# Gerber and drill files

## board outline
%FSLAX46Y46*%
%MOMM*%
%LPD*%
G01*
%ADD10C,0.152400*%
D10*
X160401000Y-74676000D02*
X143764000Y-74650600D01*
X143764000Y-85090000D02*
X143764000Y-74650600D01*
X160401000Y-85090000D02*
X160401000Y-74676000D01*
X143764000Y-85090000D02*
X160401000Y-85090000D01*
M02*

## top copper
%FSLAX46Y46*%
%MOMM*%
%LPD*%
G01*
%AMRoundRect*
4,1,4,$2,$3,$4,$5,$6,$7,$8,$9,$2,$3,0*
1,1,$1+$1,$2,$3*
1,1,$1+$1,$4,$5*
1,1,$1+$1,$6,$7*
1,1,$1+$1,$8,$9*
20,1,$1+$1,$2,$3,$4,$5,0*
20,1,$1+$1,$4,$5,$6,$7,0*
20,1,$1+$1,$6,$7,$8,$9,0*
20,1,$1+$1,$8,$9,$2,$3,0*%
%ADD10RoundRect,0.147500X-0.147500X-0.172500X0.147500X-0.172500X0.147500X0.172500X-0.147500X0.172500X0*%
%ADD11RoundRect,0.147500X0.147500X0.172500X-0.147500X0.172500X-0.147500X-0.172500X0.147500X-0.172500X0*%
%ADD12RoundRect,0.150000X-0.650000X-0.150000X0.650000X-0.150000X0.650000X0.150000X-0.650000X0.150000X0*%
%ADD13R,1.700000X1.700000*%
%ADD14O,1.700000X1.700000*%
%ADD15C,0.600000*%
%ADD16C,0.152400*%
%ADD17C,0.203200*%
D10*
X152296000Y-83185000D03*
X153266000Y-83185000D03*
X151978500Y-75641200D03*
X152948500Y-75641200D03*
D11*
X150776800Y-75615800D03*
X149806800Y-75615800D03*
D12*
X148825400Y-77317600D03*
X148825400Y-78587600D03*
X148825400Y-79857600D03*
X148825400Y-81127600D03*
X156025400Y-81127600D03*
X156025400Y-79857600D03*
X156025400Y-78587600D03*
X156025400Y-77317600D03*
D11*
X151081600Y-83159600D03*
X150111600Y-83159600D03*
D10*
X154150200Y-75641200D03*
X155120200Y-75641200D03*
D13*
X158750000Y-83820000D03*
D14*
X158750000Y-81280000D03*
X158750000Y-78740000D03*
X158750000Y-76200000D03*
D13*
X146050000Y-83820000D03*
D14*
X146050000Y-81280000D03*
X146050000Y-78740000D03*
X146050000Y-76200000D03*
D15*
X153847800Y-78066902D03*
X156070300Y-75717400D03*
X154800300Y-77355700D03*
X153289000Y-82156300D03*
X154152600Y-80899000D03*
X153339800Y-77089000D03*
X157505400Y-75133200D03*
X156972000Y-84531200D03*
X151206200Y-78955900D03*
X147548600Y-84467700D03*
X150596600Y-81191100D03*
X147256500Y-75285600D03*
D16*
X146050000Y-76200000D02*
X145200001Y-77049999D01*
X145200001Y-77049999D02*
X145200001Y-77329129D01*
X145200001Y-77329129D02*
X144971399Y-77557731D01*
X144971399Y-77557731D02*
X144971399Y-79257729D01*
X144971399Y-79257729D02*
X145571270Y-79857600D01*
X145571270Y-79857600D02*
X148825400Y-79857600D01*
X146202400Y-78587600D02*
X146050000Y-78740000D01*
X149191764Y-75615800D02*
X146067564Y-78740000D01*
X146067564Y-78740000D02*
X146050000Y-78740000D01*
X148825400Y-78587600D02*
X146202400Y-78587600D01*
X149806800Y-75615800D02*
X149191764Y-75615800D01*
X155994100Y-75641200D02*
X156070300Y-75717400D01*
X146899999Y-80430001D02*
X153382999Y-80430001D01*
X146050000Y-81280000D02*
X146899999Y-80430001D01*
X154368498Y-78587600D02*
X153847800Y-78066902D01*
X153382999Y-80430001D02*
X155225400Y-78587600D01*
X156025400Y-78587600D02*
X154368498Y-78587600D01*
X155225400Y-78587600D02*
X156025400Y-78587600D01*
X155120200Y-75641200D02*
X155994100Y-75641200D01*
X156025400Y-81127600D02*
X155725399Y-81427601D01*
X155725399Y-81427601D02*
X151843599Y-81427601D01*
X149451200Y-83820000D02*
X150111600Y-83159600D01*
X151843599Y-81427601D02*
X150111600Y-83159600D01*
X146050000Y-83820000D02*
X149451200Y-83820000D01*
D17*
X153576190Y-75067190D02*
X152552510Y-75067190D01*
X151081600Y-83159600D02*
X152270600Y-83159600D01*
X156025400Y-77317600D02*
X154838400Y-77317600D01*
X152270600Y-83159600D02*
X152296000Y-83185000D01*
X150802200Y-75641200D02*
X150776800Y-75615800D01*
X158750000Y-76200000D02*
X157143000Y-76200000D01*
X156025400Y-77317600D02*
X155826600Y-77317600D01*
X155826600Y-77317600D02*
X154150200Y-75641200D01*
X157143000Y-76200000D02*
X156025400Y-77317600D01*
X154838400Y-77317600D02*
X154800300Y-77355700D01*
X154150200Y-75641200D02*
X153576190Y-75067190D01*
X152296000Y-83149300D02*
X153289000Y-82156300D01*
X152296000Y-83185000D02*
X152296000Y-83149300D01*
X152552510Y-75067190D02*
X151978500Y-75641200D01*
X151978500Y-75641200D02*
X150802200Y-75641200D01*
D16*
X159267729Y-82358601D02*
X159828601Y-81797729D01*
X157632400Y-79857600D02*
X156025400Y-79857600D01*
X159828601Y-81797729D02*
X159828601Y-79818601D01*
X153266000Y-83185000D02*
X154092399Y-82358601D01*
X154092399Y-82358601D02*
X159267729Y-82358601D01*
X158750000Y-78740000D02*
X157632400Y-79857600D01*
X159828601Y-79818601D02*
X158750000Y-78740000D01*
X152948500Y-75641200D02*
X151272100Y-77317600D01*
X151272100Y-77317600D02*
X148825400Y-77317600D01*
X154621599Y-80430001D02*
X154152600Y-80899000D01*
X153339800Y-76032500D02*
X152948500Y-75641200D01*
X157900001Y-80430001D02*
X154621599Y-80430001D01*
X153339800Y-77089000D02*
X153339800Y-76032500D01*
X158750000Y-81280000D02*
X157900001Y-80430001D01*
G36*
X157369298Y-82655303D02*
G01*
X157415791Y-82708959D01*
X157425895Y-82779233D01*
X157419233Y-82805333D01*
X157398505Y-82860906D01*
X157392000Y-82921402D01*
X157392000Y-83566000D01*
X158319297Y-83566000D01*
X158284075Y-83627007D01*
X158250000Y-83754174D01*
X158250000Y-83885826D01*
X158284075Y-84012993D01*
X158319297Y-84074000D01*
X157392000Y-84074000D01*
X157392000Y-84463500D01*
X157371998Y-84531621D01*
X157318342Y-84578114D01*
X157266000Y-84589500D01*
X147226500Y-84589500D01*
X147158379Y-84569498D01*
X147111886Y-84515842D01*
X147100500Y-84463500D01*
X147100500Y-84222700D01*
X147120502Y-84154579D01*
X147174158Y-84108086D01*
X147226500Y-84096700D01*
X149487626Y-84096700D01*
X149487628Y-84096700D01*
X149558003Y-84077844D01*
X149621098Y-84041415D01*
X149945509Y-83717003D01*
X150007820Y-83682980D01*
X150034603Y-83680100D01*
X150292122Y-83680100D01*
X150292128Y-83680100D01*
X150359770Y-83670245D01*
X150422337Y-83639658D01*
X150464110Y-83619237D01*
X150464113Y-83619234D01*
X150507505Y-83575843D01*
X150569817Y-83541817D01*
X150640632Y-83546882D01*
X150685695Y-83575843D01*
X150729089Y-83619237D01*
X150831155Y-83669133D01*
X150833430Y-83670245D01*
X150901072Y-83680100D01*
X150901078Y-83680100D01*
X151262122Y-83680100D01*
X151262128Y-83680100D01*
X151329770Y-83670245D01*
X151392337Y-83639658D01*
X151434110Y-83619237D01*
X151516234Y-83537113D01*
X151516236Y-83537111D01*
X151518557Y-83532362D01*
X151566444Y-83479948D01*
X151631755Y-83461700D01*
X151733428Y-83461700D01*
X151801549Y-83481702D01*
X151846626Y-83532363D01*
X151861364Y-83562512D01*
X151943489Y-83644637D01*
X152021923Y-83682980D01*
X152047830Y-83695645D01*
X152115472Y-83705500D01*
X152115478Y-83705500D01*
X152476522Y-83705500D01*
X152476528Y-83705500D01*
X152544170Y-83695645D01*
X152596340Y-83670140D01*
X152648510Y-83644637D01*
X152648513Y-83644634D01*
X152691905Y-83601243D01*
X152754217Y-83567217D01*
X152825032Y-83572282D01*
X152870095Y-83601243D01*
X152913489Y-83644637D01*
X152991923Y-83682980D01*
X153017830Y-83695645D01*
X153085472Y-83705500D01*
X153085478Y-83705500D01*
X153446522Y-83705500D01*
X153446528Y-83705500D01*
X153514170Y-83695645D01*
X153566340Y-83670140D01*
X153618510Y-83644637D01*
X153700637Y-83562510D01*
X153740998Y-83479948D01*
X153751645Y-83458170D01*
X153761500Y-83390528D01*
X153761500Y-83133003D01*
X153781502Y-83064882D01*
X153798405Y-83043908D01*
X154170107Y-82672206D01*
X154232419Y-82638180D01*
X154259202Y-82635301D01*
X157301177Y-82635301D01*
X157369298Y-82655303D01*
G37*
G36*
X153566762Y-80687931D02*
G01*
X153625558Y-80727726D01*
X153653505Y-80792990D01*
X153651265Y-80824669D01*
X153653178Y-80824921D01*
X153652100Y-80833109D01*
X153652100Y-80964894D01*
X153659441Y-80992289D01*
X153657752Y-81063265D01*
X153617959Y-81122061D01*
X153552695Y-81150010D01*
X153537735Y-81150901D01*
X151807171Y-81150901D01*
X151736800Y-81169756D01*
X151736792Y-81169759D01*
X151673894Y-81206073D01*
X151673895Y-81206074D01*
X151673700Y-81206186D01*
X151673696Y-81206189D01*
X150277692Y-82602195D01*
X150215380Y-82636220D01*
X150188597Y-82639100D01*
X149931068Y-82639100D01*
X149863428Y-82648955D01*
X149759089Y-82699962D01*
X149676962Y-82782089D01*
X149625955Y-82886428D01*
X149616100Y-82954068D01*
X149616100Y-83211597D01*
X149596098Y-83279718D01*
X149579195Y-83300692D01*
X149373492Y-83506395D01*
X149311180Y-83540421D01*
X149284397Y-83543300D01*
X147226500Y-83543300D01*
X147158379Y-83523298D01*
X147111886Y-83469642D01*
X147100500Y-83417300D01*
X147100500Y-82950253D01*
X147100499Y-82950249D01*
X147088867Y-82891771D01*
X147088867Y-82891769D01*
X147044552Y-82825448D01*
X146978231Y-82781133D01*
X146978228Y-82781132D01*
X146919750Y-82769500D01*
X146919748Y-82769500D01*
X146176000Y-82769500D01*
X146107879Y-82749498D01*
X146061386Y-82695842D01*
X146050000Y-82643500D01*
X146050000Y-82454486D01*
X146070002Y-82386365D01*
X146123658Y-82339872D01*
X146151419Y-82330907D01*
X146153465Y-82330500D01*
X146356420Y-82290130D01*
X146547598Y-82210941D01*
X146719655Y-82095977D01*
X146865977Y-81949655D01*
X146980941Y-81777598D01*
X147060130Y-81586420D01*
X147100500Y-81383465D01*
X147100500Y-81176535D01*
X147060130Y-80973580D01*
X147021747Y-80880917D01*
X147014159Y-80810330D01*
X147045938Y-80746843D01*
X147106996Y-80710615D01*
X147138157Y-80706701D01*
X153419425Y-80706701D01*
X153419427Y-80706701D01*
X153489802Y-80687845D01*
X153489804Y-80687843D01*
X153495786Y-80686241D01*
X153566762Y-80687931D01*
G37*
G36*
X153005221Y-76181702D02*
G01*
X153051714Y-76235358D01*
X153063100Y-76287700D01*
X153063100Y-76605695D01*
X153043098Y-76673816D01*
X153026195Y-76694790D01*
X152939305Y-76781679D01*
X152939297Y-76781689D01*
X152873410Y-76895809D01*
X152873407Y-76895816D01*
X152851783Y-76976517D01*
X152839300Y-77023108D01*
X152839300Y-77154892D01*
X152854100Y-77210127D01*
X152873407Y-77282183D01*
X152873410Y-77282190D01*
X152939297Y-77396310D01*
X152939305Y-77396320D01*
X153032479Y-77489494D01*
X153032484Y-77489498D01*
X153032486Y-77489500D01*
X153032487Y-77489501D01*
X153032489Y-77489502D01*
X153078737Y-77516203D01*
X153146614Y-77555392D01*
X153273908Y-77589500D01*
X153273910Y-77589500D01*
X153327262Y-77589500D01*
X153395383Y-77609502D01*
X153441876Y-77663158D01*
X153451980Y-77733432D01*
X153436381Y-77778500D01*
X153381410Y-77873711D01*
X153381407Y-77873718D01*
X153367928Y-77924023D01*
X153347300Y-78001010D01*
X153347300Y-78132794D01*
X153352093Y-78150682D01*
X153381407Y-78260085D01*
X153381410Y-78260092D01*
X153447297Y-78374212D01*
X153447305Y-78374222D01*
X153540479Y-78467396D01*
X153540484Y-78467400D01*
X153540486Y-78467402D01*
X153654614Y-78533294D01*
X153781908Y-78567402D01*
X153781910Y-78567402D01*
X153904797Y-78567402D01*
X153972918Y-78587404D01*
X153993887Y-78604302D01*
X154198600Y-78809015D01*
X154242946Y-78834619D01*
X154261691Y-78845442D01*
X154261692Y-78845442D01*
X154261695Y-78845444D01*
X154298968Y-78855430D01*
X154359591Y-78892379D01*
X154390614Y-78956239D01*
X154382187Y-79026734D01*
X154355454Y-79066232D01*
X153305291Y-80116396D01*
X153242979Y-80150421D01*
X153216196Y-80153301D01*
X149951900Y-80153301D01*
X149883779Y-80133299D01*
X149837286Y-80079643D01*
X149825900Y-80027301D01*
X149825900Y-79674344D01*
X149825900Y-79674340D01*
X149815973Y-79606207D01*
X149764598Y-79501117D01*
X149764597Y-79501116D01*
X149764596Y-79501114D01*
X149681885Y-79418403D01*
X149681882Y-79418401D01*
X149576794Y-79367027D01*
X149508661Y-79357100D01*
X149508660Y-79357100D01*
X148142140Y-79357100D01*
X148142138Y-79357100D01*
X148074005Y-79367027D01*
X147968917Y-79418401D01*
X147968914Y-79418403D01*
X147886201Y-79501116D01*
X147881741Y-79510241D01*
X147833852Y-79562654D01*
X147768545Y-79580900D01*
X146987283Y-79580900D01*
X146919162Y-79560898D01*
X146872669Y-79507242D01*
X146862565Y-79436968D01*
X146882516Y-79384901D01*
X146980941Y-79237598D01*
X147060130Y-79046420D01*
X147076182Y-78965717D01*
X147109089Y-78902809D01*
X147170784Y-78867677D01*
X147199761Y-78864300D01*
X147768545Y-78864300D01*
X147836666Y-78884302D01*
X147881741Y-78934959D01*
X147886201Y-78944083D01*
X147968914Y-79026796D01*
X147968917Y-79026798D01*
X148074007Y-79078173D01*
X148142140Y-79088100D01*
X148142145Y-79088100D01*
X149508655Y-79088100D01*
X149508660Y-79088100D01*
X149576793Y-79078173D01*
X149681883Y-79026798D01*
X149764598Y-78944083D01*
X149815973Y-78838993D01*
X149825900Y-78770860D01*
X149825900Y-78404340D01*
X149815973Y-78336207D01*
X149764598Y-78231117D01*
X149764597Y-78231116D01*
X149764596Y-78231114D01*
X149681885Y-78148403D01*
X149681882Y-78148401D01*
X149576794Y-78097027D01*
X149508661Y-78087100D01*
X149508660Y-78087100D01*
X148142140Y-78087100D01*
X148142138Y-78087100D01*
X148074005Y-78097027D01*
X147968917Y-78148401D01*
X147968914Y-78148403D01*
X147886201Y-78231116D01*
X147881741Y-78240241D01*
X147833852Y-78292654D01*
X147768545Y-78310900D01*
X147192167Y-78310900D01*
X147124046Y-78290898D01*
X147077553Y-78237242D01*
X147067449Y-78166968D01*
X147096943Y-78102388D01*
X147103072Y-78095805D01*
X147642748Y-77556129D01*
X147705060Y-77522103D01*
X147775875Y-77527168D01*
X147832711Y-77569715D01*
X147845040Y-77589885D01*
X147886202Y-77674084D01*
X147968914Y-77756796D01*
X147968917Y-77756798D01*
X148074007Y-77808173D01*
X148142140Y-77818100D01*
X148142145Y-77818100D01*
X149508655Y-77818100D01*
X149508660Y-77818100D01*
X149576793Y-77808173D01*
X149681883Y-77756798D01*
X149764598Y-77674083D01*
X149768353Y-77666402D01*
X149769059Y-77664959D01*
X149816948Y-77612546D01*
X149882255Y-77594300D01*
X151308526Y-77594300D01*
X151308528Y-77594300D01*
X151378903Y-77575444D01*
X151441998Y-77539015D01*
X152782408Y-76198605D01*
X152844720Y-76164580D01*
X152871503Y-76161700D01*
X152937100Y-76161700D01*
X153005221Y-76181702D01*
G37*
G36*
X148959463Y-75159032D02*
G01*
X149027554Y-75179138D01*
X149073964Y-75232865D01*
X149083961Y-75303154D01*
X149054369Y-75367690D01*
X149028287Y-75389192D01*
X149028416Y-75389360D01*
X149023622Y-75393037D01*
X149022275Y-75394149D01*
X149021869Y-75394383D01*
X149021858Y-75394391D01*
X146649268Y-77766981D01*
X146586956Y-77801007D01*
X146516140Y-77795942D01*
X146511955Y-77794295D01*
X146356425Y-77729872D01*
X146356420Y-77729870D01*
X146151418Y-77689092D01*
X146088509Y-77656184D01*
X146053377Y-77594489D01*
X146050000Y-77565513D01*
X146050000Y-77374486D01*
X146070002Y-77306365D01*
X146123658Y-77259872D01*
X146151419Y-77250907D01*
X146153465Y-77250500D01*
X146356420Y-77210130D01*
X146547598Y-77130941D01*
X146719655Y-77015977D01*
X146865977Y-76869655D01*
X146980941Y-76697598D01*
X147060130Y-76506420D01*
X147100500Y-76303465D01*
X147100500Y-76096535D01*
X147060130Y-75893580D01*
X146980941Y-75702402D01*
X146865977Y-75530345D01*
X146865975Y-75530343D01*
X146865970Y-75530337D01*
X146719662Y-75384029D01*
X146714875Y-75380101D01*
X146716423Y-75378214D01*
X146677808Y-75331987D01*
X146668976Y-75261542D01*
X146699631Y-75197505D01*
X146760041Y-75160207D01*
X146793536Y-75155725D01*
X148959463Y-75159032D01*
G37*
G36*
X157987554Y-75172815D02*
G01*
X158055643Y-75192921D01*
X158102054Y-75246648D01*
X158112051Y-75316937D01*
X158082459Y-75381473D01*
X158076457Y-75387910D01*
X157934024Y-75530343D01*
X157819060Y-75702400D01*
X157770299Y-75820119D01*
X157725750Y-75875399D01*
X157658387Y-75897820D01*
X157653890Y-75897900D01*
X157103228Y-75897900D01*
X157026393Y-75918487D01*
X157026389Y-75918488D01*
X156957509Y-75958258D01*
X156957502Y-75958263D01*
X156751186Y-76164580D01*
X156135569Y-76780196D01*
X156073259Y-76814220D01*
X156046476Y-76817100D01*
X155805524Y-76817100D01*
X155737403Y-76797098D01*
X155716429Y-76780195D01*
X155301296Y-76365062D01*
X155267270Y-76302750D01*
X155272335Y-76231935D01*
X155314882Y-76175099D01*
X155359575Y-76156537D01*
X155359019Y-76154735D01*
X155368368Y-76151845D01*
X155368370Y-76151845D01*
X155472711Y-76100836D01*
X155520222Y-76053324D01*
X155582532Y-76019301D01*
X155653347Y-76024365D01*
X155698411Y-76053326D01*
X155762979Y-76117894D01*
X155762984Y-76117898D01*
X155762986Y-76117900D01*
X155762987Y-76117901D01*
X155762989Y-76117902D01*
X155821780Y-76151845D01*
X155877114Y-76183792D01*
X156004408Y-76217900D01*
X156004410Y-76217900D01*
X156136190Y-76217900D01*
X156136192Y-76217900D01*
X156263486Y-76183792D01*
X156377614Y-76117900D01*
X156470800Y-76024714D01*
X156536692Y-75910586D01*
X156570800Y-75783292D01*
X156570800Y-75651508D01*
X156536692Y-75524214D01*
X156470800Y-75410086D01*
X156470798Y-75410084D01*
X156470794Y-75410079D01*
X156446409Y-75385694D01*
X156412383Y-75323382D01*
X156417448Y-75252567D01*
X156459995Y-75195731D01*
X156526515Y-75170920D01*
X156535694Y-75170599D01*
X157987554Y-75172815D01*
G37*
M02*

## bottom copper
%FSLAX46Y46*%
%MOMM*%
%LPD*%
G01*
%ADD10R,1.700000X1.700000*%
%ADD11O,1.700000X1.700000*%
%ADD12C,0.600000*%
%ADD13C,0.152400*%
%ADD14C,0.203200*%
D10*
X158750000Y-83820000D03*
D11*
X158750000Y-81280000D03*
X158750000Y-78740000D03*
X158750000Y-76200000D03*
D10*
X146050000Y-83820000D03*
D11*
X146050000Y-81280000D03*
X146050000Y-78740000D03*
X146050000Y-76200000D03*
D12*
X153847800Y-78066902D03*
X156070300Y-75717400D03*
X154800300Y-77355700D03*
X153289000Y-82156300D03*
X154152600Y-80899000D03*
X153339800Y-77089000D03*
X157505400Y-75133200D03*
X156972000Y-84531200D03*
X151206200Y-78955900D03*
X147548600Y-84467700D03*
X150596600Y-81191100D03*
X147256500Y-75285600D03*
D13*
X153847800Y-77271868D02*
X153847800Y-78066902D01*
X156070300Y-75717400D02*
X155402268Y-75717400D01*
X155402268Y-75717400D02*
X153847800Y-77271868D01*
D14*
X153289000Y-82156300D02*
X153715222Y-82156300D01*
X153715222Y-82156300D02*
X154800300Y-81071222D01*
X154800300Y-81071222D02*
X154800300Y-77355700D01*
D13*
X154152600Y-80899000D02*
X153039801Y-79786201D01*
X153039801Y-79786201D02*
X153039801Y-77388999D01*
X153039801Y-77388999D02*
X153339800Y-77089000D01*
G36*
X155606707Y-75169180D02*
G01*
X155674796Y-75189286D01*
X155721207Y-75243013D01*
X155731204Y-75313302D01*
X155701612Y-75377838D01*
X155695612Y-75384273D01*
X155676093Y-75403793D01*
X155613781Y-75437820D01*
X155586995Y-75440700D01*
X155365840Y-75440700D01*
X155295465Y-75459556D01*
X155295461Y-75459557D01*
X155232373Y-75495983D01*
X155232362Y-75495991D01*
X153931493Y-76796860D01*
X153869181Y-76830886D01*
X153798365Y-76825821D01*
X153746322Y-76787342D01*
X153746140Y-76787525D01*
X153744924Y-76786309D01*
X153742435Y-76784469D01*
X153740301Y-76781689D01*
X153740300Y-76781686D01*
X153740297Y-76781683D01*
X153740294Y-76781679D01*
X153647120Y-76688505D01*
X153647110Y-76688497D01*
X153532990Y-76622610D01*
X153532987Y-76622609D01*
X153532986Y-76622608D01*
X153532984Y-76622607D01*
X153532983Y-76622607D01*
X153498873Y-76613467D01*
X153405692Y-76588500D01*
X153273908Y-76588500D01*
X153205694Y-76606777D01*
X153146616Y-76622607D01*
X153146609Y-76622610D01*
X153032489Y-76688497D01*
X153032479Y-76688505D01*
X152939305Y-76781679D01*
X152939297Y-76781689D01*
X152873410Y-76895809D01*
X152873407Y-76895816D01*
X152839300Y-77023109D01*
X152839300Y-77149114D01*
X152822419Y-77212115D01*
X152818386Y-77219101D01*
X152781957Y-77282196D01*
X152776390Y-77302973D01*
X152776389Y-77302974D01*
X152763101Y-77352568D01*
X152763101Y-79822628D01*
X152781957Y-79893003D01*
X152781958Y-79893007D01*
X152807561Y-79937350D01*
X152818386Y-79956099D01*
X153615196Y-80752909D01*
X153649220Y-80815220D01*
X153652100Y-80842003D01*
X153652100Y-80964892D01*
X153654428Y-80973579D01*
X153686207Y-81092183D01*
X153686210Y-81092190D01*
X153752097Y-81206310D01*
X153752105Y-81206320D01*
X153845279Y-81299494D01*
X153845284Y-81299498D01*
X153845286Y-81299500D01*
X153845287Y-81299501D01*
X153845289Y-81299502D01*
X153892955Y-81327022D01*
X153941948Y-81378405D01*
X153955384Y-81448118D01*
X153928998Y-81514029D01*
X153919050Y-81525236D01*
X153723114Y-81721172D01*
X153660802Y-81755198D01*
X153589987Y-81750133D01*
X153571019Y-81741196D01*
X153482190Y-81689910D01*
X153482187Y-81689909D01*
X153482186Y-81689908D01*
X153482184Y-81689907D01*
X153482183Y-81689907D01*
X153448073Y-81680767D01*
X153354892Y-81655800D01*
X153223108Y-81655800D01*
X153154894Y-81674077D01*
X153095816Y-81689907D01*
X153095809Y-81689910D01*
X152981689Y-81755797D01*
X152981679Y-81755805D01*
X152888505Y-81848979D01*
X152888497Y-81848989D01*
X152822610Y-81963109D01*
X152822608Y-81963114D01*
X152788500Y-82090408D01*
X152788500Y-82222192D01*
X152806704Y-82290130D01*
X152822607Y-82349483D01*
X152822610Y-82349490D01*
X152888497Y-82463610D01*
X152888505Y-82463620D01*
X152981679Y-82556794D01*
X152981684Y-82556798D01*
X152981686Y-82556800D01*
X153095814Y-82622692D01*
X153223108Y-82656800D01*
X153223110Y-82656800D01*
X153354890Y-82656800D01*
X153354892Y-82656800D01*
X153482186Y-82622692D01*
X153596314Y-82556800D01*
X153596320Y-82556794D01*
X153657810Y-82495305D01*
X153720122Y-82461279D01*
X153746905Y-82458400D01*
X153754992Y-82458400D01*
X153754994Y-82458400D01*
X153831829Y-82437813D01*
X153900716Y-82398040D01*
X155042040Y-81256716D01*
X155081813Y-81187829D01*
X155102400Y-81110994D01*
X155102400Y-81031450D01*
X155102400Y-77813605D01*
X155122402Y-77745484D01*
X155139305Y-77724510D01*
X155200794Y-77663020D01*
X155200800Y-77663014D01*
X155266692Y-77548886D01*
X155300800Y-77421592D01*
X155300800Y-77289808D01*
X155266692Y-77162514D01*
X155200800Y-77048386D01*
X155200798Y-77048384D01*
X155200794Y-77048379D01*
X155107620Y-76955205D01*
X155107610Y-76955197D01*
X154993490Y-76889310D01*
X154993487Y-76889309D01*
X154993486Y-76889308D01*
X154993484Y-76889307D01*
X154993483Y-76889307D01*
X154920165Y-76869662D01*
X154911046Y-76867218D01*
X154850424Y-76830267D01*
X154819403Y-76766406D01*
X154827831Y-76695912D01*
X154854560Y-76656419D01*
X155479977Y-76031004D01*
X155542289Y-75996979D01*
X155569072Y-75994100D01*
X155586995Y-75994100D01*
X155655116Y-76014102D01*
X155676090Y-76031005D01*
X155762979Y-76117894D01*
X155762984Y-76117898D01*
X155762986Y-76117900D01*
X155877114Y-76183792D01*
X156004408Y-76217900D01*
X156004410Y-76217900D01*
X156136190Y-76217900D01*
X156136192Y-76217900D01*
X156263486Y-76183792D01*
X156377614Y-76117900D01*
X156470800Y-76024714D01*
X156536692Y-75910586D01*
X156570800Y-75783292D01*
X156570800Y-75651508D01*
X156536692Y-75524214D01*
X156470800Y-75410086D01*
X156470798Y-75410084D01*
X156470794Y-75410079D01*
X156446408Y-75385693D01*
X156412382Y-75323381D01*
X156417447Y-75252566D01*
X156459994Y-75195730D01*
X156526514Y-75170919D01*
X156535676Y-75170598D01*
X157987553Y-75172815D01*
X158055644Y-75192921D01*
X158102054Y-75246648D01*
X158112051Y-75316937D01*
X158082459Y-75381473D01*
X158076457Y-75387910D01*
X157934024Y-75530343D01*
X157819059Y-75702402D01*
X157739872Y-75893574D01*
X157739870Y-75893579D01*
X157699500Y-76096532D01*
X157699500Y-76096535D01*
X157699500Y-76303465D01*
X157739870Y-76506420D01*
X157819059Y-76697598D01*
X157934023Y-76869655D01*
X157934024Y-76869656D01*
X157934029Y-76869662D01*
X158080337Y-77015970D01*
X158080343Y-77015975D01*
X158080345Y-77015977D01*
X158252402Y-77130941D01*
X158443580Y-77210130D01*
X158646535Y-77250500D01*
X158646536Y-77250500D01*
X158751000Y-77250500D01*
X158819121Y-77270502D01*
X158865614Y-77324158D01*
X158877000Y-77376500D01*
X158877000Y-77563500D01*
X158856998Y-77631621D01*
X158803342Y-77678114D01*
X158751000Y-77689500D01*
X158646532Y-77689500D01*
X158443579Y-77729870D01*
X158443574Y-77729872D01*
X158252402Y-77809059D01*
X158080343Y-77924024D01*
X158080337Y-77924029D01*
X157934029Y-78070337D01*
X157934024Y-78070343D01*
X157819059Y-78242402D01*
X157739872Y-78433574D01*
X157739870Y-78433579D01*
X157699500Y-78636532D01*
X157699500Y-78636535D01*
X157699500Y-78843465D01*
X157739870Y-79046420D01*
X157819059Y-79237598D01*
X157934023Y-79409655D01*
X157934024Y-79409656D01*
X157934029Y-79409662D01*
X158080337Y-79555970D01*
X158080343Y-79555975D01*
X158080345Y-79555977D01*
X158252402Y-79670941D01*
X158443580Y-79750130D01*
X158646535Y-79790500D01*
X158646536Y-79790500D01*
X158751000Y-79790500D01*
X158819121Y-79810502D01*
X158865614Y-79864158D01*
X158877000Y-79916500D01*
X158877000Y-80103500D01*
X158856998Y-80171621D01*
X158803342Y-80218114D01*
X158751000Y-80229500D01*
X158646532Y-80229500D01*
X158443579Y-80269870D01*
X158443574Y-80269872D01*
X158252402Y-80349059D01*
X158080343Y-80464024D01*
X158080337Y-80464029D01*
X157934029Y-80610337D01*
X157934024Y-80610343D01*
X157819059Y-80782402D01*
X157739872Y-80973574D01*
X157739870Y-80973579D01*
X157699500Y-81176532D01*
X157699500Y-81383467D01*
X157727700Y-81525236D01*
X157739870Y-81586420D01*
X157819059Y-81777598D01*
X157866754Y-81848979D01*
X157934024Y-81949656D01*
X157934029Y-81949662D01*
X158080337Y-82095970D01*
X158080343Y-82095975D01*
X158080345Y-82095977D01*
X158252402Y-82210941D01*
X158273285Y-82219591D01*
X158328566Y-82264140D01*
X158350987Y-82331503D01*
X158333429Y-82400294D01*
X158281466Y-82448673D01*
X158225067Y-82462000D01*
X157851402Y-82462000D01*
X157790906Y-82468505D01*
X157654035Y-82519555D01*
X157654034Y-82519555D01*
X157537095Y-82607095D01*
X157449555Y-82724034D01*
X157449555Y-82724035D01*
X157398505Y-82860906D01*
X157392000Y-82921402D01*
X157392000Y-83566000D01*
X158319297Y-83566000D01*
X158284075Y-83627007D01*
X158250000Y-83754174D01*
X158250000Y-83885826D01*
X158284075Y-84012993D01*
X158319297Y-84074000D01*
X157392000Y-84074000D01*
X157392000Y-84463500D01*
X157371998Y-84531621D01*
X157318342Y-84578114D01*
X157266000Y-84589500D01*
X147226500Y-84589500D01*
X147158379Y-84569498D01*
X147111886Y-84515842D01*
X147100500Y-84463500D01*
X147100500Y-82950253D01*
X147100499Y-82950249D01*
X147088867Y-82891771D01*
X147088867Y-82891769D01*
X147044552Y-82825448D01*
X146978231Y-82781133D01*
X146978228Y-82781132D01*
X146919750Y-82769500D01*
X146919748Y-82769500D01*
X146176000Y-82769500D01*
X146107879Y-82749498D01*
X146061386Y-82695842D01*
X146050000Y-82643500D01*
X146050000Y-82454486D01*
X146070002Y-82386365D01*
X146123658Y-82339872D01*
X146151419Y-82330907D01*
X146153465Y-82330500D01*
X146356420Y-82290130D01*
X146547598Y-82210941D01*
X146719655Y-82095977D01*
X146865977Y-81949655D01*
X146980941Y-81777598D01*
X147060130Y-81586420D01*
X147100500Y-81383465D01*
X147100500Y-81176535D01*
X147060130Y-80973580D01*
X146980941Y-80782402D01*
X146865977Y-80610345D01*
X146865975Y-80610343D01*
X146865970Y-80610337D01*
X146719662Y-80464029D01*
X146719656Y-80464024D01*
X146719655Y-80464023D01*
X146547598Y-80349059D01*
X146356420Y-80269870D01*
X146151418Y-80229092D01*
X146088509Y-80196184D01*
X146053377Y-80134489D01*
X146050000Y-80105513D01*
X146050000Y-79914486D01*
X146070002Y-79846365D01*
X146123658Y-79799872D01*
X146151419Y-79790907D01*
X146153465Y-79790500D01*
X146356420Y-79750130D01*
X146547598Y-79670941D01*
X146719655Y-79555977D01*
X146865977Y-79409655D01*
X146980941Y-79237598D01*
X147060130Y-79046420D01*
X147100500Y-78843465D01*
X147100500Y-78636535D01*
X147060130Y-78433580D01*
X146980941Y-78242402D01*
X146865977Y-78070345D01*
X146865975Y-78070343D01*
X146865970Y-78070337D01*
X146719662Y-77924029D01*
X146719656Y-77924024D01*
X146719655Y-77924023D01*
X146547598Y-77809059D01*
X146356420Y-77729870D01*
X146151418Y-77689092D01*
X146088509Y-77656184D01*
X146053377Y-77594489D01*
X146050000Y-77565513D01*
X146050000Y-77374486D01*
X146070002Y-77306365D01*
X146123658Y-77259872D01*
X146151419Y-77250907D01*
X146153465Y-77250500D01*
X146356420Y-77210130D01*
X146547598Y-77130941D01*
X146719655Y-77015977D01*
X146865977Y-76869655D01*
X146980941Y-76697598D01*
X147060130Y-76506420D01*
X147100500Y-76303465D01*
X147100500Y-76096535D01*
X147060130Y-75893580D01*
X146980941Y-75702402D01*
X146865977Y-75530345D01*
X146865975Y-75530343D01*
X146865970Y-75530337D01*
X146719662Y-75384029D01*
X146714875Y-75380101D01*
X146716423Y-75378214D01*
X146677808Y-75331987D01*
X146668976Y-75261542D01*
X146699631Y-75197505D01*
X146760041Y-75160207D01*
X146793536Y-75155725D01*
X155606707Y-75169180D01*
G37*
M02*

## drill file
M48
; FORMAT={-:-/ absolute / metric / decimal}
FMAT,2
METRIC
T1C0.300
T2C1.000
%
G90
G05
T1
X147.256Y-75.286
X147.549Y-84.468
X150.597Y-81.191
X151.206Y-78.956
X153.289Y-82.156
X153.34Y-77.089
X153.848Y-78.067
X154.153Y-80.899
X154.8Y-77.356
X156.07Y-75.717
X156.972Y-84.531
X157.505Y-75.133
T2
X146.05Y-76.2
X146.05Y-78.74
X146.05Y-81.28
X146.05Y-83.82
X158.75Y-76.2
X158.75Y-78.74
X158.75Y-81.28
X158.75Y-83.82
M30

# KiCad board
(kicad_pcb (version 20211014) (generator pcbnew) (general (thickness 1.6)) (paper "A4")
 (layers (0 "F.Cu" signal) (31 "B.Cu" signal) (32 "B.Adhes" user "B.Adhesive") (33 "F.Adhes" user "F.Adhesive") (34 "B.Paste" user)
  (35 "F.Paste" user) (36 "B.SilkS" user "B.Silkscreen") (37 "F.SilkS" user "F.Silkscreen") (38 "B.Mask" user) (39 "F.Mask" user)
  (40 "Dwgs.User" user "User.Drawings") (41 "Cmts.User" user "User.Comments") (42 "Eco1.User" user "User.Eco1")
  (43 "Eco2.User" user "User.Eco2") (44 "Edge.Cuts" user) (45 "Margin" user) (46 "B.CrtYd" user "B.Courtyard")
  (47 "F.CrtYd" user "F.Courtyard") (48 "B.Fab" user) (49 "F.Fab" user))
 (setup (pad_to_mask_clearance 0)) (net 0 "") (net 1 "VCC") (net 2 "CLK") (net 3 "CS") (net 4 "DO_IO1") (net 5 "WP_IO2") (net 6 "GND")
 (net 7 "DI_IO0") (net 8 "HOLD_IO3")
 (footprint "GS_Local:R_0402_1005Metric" (layer "F.Cu") (at 152.781 83.185)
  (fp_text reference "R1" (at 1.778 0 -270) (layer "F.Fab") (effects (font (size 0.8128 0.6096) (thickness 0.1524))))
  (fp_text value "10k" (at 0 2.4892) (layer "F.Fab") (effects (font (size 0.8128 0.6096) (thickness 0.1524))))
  (pad "1" smd roundrect locked (at -0.485 0) (size 0.59 0.64) (layers "F.Cu" "F.Paste" "F.Mask") (roundrect_rratio 0.25) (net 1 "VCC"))
  (pad "2" smd roundrect locked (at 0.485 0) (size 0.59 0.64) (layers "F.Cu" "F.Paste" "F.Mask") (roundrect_rratio 0.25) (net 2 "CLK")))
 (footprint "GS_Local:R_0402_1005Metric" (layer "F.Cu") (at 152.4635 75.6412)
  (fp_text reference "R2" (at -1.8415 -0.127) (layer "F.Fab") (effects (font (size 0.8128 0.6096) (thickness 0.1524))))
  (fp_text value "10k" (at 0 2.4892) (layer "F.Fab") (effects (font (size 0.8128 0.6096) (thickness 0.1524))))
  (pad "1" smd roundrect locked (at -0.485 0) (size 0.59 0.64) (layers "F.Cu" "F.Paste" "F.Mask") (roundrect_rratio 0.25) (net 1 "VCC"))
  (pad "2" smd roundrect locked (at 0.485 0) (size 0.59 0.64) (layers "F.Cu" "F.Paste" "F.Mask") (roundrect_rratio 0.25) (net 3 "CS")))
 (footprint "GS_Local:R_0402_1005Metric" (layer "F.Cu") (at 150.2918 75.6158 180)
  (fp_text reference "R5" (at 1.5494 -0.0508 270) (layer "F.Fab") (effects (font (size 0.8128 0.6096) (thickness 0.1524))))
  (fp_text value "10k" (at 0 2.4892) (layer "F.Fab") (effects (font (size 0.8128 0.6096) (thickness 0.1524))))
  (pad "1" smd roundrect locked (at -0.485 0 180) (size 0.59 0.64) (layers "F.Cu" "F.Paste" "F.Mask") (roundrect_rratio 0.25) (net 1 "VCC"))
  (pad "2" smd roundrect locked (at 0.485 0 180) (size 0.59 0.64) (layers "F.Cu" "F.Paste" "F.Mask") (roundrect_rratio 0.25)
   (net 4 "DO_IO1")))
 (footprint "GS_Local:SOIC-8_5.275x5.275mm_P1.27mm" (layer "F.Cu") (at 152.4254 79.2226)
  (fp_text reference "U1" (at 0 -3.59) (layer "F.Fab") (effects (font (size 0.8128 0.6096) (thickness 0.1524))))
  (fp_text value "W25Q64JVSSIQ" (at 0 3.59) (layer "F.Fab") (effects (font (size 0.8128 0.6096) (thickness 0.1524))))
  (pad "1" smd roundrect locked (at -3.6 -1.905) (size 1.6 0.6) (layers "F.Cu" "F.Paste" "F.Mask") (roundrect_rratio 0.25) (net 3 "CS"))
  (pad "2" smd roundrect locked (at -3.6 -0.635) (size 1.6 0.6) (layers "F.Cu" "F.Paste" "F.Mask") (roundrect_rratio 0.25) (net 4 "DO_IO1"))
  (pad "3" smd roundrect locked (at -3.6 0.635) (size 1.6 0.6) (layers "F.Cu" "F.Paste" "F.Mask") (roundrect_rratio 0.25) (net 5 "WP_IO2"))
  (pad "4" smd roundrect locked (at -3.6 1.905) (size 1.6 0.6) (layers "F.Cu" "F.Paste" "F.Mask") (roundrect_rratio 0.25) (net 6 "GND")
   (zone_connect 2))
  (pad "5" smd roundrect locked (at 3.6 1.905) (size 1.6 0.6) (layers "F.Cu" "F.Paste" "F.Mask") (roundrect_rratio 0.25) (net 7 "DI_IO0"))
  (pad "6" smd roundrect locked (at 3.6 0.635) (size 1.6 0.6) (layers "F.Cu" "F.Paste" "F.Mask") (roundrect_rratio 0.25) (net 2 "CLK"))
  (pad "7" smd roundrect locked (at 3.6 -0.635) (size 1.6 0.6) (layers "F.Cu" "F.Paste" "F.Mask") (roundrect_rratio 0.25) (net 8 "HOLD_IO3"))
  (pad "8" smd roundrect locked (at 3.6 -1.905) (size 1.6 0.6) (layers "F.Cu" "F.Paste" "F.Mask") (roundrect_rratio 0.25) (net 1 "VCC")))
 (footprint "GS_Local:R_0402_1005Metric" (layer "F.Cu") (at 150.5966 83.1596 180)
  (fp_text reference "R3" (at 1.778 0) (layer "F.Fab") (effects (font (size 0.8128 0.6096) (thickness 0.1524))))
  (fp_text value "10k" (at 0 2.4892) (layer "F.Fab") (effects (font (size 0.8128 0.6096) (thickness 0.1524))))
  (pad "1" smd roundrect locked (at -0.485 0 180) (size 0.59 0.64) (layers "F.Cu" "F.Paste" "F.Mask") (roundrect_rratio 0.25) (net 1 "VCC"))
  (pad "2" smd roundrect locked (at 0.485 0 180) (size 0.59 0.64) (layers "F.Cu" "F.Paste" "F.Mask") (roundrect_rratio 0.25)
   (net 7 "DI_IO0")))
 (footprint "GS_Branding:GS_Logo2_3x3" (layer "F.Cu") (at 155.4734 83.566)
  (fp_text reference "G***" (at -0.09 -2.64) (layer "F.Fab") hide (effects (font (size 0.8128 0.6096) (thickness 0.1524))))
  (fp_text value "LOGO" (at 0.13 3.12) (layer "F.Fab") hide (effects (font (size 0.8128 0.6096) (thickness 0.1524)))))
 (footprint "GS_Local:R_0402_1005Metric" (layer "F.Cu") (at 154.6352 75.6412)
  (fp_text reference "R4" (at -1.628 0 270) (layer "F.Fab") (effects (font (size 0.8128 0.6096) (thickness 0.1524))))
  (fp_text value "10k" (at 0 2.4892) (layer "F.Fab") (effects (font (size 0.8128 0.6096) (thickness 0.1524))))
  (pad "1" smd roundrect locked (at -0.485 0) (size 0.59 0.64) (layers "F.Cu" "F.Paste" "F.Mask") (roundrect_rratio 0.25) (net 1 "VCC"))
  (pad "2" smd roundrect locked (at 0.485 0) (size 0.59 0.64) (layers "F.Cu" "F.Paste" "F.Mask") (roundrect_rratio 0.25) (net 8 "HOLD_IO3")))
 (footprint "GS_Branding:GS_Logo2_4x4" (layer "B.Cu") (at 152.2603 79.9211 180)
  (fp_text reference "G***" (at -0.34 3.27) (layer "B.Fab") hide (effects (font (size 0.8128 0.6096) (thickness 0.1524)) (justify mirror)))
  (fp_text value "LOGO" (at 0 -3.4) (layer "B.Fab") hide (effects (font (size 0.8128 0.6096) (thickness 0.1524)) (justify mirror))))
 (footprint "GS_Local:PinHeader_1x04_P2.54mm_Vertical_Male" (layer "B.Cu") (at 158.75 83.82)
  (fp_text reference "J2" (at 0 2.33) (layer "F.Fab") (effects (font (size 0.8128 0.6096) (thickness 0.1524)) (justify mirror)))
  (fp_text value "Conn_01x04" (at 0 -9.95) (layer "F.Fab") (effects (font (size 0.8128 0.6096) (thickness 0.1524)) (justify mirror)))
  (pad "1" thru_hole rect locked (at 0 0) (size 1.7 1.7) (drill 1) (layers *.Cu *.Mask) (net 6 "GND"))
  (pad "2" thru_hole oval locked (at 0 -2.54) (size 1.7 1.7) (drill 1) (layers *.Cu *.Mask) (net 3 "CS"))
  (pad "3" thru_hole oval locked (at 0 -5.08) (size 1.7 1.7) (drill 1) (layers *.Cu *.Mask) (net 2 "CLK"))
  (pad "4" thru_hole oval locked (at 0 -7.62) (size 1.7 1.7) (drill 1) (layers *.Cu *.Mask) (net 1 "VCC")))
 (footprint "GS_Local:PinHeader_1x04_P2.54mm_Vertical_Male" (layer "B.Cu") (at 146.05 83.82)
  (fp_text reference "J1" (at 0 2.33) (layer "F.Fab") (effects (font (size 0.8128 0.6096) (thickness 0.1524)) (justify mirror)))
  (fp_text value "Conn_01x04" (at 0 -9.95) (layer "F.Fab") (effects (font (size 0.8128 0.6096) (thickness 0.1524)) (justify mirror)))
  (pad "1" thru_hole rect locked (at 0 0) (size 1.7 1.7) (drill 1) (layers *.Cu *.Mask) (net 7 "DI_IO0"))
  (pad "2" thru_hole oval locked (at 0 -2.54) (size 1.7 1.7) (drill 1) (layers *.Cu *.Mask) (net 8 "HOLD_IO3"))
  (pad "3" thru_hole oval locked (at 0 -5.08) (size 1.7 1.7) (drill 1) (layers *.Cu *.Mask) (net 4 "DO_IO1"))
  (pad "4" thru_hole oval locked (at 0 -7.62) (size 1.7 1.7) (drill 1) (layers *.Cu *.Mask) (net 5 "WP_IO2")))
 (gr_line (start 160.401 74.676) (end 143.764 74.6506) (layer "Edge.Cuts") (width 0.1524))
 (gr_line (start 143.764 85.09) (end 143.764 74.6506) (layer "Edge.Cuts") (width 0.1524))
 (gr_line (start 160.401 85.09) (end 160.401 74.676) (layer "Edge.Cuts") (width 0.1524))
 (gr_line (start 143.764 85.09) (end 160.401 85.09) (layer "Edge.Cuts") (width 0.1524))
 (segment (start 146.05 76.2) (end 145.200001 77.049999) (width 0.1524) (layer "F.Cu") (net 5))
 (segment (start 145.200001 77.049999) (end 145.200001 77.329129) (width 0.1524) (layer "F.Cu") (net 5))
 (segment (start 145.200001 77.329129) (end 144.971399 77.557731) (width 0.1524) (layer "F.Cu") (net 5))
 (segment (start 144.971399 77.557731) (end 144.971399 79.257729) (width 0.1524) (layer "F.Cu") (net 5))
 (segment (start 144.971399 79.257729) (end 145.57127 79.8576) (width 0.1524) (layer "F.Cu") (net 5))
 (segment (start 145.57127 79.8576) (end 148.8254 79.8576) (width 0.1524) (layer "F.Cu") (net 5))
 (segment (start 146.2024 78.5876) (end 146.05 78.74) (width 0.1524) (layer "F.Cu") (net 4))
 (segment (start 149.191764 75.6158) (end 146.067564 78.74) (width 0.1524) (layer "F.Cu") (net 4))
 (segment (start 146.067564 78.74) (end 146.05 78.74) (width 0.1524) (layer "F.Cu") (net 4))
 (segment (start 148.8254 78.5876) (end 146.2024 78.5876) (width 0.1524) (layer "F.Cu") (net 4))
 (segment (start 149.8068 75.6158) (end 149.191764 75.6158) (width 0.1524) (layer "F.Cu") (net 4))
 (segment (start 155.9941 75.6412) (end 156.0703 75.7174) (width 0.1524) (layer "F.Cu") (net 8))
 (segment (start 146.899999 80.430001) (end 153.382999 80.430001) (width 0.1524) (layer "F.Cu") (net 8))
 (segment (start 146.05 81.28) (end 146.899999 80.430001) (width 0.1524) (layer "F.Cu") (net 8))
 (segment (start 154.368498 78.5876) (end 153.8478 78.066902) (width 0.1524) (layer "F.Cu") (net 8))
 (segment (start 153.382999 80.430001) (end 155.2254 78.5876) (width 0.1524) (layer "F.Cu") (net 8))
 (segment (start 156.0254 78.5876) (end 154.368498 78.5876) (width 0.1524) (layer "F.Cu") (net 8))
 (segment (start 155.2254 78.5876) (end 156.0254 78.5876) (width 0.1524) (layer "F.Cu") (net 8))
 (segment (start 155.1202 75.6412) (end 155.9941 75.6412) (width 0.1524) (layer "F.Cu") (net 8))
 (via (at 153.8478 78.066902) (size 0.6) (drill 0.3) (layers "F.Cu" "B.Cu") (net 8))
 (via (at 156.0703 75.7174) (size 0.6) (drill 0.3) (layers "F.Cu" "B.Cu") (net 8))
 (segment (start 153.8478 77.271868) (end 153.8478 78.066902) (width 0.1524) (layer "B.Cu") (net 8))
 (segment (start 156.0703 75.7174) (end 155.402268 75.7174) (width 0.1524) (layer "B.Cu") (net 8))
 (segment (start 155.402268 75.7174) (end 153.8478 77.271868) (width 0.1524) (layer "B.Cu") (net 8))
 (segment (start 156.0254 81.1276) (end 155.725399 81.427601) (width 0.1524) (layer "F.Cu") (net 7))
 (segment (start 155.725399 81.427601) (end 151.843599 81.427601) (width 0.1524) (layer "F.Cu") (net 7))
 (segment (start 149.4512 83.82) (end 150.1116 83.1596) (width 0.1524) (layer "F.Cu") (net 7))
 (segment (start 151.843599 81.427601) (end 150.1116 83.1596) (width 0.1524) (layer "F.Cu") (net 7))
 (segment (start 146.05 83.82) (end 149.4512 83.82) (width 0.1524) (layer "F.Cu") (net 7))
 (segment (start 153.57619 75.06719) (end 152.55251 75.06719) (width 0.2032) (layer "F.Cu") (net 1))
 (segment (start 151.0816 83.1596) (end 152.2706 83.1596) (width 0.2032) (layer "F.Cu") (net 1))
 (segment (start 156.0254 77.3176) (end 154.8384 77.3176) (width 0.2032) (layer "F.Cu") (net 1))
 (segment (start 152.2706 83.1596) (end 152.296 83.185) (width 0.2032) (layer "F.Cu") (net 1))
 (segment (start 150.8022 75.6412) (end 150.7768 75.6158) (width 0.2032) (layer "F.Cu") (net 1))
 (segment (start 158.75 76.2) (end 157.143 76.2) (width 0.2032) (layer "F.Cu") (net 1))
 (segment (start 156.0254 77.3176) (end 155.8266 77.3176) (width 0.2032) (layer "F.Cu") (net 1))
 (segment (start 155.8266 77.3176) (end 154.1502 75.6412) (width 0.2032) (layer "F.Cu") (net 1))
 (segment (start 157.143 76.2) (end 156.0254 77.3176) (width 0.2032) (layer "F.Cu") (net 1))
 (segment (start 154.8384 77.3176) (end 154.8003 77.3557) (width 0.2032) (layer "F.Cu") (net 1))
 (segment (start 154.1502 75.6412) (end 153.57619 75.06719) (width 0.2032) (layer "F.Cu") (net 1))
 (segment (start 152.296 83.1493) (end 153.289 82.1563) (width 0.2032) (layer "F.Cu") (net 1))
 (segment (start 152.296 83.185) (end 152.296 83.1493) (width 0.2032) (layer "F.Cu") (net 1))
 (segment (start 152.55251 75.06719) (end 151.9785 75.6412) (width 0.2032) (layer "F.Cu") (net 1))
 (segment (start 151.9785 75.6412) (end 150.8022 75.6412) (width 0.2032) (layer "F.Cu") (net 1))
 (via (at 154.8003 77.3557) (size 0.6) (drill 0.3) (layers "F.Cu" "B.Cu") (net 1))
 (via (at 153.289 82.1563) (size 0.6) (drill 0.3) (layers "F.Cu" "B.Cu") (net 1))
 (segment (start 153.289 82.1563) (end 153.715222 82.1563) (width 0.2032) (layer "B.Cu") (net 1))
 (segment (start 153.715222 82.1563) (end 154.8003 81.071222) (width 0.2032) (layer "B.Cu") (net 1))
 (segment (start 154.8003 81.071222) (end 154.8003 77.3557) (width 0.2032) (layer "B.Cu") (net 1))
 (segment (start 159.267729 82.358601) (end 159.828601 81.797729) (width 0.1524) (layer "F.Cu") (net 2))
 (segment (start 157.6324 79.8576) (end 156.0254 79.8576) (width 0.1524) (layer "F.Cu") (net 2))
 (segment (start 159.828601 81.797729) (end 159.828601 79.818601) (width 0.1524) (layer "F.Cu") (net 2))
 (segment (start 153.266 83.185) (end 154.092399 82.358601) (width 0.1524) (layer "F.Cu") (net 2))
 (segment (start 154.092399 82.358601) (end 159.267729 82.358601) (width 0.1524) (layer "F.Cu") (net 2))
 (segment (start 158.75 78.74) (end 157.6324 79.8576) (width 0.1524) (layer "F.Cu") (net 2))
 (segment (start 159.828601 79.818601) (end 158.75 78.74) (width 0.1524) (layer "F.Cu") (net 2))
 (segment (start 152.9485 75.6412) (end 151.2721 77.3176) (width 0.1524) (layer "F.Cu") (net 3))
 (segment (start 151.2721 77.3176) (end 148.8254 77.3176) (width 0.1524) (layer "F.Cu") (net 3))
 (segment (start 154.621599 80.430001) (end 154.1526 80.899) (width 0.1524) (layer "F.Cu") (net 3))
 (segment (start 153.3398 76.0325) (end 152.9485 75.6412) (width 0.1524) (layer "F.Cu") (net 3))
 (segment (start 157.900001 80.430001) (end 154.621599 80.430001) (width 0.1524) (layer "F.Cu") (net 3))
 (segment (start 153.3398 77.089) (end 153.3398 76.0325) (width 0.1524) (layer "F.Cu") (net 3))
 (segment (start 158.75 81.28) (end 157.900001 80.430001) (width 0.1524) (layer "F.Cu") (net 3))
 (via (at 154.1526 80.899) (size 0.6) (drill 0.3) (layers "F.Cu" "B.Cu") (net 3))
 (via (at 153.3398 77.089) (size 0.6) (drill 0.3) (layers "F.Cu" "B.Cu") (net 3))
 (segment (start 154.1526 80.899) (end 153.039801 79.786201) (width 0.1524) (layer "B.Cu") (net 3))
 (segment (start 153.039801 79.786201) (end 153.039801 77.388999) (width 0.1524) (layer "B.Cu") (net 3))
 (segment (start 153.039801 77.388999) (end 153.3398 77.089) (width 0.1524) (layer "B.Cu") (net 3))
 (via (at 157.5054 75.1332) (size 0.6) (drill 0.3) (layers "F.Cu" "B.Cu") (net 6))
 (via (at 156.972 84.5312) (size 0.6) (drill 0.3) (layers "F.Cu" "B.Cu") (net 6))
 (via (at 151.2062 78.9559) (size 0.6) (drill 0.3) (layers "F.Cu" "B.Cu") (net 6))
 (via (at 147.5486 84.4677) (size 0.6) (drill 0.3) (layers "F.Cu" "B.Cu") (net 6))
 (via (at 150.5966 81.1911) (size 0.6) (drill 0.3) (layers "F.Cu" "B.Cu") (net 6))
 (via (at 147.2565 75.2856) (size 0.6) (drill 0.3) (layers "F.Cu" "B.Cu") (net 6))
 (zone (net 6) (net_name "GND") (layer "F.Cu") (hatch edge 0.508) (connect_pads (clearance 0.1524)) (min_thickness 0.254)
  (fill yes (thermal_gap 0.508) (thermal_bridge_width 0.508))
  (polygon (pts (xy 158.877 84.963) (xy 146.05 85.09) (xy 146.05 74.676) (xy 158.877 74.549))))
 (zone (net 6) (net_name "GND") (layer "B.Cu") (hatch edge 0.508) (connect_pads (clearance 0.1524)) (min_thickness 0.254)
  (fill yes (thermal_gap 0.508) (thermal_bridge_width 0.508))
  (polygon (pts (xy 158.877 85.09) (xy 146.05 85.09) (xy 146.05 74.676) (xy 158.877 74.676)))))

